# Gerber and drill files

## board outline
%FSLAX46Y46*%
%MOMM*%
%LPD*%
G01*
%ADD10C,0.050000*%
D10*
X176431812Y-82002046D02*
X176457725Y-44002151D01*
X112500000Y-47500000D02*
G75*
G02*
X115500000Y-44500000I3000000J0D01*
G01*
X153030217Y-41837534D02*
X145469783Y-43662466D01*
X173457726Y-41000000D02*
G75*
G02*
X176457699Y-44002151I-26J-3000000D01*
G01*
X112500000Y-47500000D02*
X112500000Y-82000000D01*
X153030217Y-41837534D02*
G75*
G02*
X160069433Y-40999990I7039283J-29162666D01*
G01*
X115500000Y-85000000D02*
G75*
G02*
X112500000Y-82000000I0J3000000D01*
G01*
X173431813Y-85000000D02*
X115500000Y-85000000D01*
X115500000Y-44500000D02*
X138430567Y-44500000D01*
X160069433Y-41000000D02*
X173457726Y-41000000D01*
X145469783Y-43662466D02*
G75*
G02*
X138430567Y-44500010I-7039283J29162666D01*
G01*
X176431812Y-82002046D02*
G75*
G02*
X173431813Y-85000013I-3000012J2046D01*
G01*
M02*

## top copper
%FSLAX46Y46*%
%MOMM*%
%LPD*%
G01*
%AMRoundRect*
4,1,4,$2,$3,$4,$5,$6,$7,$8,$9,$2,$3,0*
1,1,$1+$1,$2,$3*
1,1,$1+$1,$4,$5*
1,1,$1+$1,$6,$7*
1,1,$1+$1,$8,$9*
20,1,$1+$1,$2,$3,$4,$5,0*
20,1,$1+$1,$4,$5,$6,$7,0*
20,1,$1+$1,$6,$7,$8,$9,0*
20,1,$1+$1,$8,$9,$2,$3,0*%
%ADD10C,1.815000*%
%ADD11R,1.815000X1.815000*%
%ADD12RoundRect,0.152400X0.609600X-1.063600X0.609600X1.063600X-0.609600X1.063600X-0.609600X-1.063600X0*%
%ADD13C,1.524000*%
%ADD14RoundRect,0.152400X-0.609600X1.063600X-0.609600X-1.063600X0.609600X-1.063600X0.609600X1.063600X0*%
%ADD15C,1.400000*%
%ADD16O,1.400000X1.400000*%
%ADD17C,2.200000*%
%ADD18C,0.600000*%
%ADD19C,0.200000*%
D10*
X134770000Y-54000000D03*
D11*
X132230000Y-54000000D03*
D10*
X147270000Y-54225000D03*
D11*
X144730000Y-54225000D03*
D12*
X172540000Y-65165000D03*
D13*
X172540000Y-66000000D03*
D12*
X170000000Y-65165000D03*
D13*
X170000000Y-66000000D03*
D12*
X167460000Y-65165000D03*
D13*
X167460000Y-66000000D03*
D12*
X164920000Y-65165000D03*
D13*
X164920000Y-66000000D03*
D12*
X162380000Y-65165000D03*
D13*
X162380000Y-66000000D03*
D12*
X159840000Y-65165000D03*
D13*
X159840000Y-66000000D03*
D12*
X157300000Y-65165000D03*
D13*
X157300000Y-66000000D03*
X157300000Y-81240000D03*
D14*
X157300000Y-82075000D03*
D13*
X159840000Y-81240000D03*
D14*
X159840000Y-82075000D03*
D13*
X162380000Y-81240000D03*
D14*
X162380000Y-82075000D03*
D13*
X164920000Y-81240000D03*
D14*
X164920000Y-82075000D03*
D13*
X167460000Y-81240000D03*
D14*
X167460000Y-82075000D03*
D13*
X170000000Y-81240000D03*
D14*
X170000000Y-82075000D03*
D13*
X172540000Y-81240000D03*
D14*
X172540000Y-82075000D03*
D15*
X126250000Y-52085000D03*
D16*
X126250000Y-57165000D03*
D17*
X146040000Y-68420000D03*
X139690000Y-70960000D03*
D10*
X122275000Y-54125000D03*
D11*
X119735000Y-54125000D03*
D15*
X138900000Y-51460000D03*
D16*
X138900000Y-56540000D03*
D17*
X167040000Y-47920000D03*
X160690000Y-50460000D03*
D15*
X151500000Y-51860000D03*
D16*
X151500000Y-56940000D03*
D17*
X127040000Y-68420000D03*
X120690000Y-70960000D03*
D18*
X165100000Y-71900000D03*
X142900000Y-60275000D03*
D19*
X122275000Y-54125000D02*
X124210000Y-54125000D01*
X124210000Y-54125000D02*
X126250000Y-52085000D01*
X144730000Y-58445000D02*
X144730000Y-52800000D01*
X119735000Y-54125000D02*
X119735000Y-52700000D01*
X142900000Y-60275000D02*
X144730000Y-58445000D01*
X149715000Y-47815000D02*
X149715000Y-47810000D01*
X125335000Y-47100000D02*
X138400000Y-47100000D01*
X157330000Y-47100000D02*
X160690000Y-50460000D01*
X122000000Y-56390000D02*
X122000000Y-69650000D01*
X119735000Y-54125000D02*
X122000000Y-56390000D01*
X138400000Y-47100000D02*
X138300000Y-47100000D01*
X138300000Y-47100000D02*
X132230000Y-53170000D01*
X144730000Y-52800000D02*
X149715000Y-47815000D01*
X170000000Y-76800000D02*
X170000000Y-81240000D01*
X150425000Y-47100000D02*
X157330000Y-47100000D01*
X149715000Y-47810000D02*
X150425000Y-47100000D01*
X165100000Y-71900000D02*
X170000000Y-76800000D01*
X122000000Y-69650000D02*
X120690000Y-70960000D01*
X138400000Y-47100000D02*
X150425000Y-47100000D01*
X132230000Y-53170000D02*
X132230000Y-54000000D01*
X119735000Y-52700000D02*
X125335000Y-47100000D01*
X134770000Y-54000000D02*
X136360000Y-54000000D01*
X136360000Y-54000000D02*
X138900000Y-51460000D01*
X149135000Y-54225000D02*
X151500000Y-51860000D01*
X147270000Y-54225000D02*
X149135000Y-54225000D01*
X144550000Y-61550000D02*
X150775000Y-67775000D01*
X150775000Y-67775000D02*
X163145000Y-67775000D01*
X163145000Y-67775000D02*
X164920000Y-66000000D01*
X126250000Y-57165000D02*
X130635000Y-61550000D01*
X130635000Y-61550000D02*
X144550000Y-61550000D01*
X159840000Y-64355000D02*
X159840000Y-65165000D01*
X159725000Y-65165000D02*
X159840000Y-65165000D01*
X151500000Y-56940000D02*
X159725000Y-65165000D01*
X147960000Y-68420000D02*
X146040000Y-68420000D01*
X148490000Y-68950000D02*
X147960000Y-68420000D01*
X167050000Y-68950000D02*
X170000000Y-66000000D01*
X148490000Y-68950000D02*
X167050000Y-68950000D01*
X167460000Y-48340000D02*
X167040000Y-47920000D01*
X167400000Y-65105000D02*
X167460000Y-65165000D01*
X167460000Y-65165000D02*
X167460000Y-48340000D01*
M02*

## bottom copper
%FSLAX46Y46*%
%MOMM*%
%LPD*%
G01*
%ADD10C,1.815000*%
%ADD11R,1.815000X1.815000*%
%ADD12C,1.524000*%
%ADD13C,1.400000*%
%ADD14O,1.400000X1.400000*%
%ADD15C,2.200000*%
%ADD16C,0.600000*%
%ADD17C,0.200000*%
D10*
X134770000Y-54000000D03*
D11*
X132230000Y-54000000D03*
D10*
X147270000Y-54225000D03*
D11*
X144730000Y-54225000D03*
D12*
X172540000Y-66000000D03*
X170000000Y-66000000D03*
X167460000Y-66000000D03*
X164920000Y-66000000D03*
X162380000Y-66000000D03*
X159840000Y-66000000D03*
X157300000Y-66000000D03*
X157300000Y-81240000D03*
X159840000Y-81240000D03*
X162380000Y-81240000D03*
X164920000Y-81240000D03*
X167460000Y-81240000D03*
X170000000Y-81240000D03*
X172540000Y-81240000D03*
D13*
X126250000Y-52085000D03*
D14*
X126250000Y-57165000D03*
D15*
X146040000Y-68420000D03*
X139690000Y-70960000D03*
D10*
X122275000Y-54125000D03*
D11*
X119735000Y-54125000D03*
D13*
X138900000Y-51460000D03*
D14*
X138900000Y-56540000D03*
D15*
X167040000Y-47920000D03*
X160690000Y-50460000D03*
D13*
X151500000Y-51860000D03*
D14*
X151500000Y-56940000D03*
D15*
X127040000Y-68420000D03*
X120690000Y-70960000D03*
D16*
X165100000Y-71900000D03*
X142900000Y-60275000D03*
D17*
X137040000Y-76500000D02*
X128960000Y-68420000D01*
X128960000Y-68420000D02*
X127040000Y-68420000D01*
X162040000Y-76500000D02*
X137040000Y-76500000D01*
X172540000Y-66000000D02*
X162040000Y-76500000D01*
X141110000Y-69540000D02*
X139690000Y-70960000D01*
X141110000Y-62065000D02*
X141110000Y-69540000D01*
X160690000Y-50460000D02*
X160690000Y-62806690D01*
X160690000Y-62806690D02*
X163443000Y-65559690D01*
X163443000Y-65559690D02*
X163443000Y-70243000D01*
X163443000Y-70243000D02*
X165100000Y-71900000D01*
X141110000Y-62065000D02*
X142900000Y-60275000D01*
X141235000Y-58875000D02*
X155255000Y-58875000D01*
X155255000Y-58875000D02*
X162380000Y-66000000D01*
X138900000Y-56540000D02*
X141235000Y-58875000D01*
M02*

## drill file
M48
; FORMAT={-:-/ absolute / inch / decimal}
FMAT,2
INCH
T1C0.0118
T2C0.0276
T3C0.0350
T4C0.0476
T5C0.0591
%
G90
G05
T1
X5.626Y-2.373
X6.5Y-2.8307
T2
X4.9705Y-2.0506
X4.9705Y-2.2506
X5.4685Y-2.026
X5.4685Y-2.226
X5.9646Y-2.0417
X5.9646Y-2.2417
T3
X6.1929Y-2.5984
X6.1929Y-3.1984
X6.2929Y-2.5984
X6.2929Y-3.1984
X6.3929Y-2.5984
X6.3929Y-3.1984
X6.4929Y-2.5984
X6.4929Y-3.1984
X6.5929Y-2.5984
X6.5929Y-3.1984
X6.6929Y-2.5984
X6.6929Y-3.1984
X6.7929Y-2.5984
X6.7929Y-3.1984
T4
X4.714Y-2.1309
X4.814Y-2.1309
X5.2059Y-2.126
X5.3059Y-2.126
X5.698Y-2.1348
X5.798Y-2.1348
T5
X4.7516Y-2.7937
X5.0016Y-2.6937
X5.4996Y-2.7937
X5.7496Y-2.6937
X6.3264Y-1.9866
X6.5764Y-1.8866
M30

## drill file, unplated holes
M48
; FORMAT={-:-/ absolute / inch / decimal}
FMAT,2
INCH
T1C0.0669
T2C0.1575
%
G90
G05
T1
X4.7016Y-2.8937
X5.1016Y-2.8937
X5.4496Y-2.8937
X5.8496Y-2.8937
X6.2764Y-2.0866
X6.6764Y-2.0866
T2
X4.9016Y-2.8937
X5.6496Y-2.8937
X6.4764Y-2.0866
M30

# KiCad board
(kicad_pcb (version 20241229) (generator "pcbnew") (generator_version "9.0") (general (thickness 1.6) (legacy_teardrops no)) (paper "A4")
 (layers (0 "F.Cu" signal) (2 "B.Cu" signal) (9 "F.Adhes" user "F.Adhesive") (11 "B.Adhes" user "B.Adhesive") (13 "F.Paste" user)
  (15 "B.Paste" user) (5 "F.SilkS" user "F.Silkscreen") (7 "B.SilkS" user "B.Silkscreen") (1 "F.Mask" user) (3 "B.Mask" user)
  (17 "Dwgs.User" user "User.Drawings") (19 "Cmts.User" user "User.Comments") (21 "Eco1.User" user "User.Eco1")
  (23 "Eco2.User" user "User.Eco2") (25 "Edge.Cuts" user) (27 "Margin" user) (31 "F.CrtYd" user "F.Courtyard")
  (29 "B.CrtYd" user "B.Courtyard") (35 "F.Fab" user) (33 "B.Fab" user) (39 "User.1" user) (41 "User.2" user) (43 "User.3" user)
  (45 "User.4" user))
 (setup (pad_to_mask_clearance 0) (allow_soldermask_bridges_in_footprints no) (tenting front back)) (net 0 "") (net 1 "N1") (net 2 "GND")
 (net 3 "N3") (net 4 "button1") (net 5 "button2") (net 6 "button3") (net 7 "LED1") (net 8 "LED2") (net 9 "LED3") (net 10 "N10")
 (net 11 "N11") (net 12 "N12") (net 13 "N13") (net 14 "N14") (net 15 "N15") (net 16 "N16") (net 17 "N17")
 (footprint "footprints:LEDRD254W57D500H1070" (layer "F.Cu") (at 133.5 54)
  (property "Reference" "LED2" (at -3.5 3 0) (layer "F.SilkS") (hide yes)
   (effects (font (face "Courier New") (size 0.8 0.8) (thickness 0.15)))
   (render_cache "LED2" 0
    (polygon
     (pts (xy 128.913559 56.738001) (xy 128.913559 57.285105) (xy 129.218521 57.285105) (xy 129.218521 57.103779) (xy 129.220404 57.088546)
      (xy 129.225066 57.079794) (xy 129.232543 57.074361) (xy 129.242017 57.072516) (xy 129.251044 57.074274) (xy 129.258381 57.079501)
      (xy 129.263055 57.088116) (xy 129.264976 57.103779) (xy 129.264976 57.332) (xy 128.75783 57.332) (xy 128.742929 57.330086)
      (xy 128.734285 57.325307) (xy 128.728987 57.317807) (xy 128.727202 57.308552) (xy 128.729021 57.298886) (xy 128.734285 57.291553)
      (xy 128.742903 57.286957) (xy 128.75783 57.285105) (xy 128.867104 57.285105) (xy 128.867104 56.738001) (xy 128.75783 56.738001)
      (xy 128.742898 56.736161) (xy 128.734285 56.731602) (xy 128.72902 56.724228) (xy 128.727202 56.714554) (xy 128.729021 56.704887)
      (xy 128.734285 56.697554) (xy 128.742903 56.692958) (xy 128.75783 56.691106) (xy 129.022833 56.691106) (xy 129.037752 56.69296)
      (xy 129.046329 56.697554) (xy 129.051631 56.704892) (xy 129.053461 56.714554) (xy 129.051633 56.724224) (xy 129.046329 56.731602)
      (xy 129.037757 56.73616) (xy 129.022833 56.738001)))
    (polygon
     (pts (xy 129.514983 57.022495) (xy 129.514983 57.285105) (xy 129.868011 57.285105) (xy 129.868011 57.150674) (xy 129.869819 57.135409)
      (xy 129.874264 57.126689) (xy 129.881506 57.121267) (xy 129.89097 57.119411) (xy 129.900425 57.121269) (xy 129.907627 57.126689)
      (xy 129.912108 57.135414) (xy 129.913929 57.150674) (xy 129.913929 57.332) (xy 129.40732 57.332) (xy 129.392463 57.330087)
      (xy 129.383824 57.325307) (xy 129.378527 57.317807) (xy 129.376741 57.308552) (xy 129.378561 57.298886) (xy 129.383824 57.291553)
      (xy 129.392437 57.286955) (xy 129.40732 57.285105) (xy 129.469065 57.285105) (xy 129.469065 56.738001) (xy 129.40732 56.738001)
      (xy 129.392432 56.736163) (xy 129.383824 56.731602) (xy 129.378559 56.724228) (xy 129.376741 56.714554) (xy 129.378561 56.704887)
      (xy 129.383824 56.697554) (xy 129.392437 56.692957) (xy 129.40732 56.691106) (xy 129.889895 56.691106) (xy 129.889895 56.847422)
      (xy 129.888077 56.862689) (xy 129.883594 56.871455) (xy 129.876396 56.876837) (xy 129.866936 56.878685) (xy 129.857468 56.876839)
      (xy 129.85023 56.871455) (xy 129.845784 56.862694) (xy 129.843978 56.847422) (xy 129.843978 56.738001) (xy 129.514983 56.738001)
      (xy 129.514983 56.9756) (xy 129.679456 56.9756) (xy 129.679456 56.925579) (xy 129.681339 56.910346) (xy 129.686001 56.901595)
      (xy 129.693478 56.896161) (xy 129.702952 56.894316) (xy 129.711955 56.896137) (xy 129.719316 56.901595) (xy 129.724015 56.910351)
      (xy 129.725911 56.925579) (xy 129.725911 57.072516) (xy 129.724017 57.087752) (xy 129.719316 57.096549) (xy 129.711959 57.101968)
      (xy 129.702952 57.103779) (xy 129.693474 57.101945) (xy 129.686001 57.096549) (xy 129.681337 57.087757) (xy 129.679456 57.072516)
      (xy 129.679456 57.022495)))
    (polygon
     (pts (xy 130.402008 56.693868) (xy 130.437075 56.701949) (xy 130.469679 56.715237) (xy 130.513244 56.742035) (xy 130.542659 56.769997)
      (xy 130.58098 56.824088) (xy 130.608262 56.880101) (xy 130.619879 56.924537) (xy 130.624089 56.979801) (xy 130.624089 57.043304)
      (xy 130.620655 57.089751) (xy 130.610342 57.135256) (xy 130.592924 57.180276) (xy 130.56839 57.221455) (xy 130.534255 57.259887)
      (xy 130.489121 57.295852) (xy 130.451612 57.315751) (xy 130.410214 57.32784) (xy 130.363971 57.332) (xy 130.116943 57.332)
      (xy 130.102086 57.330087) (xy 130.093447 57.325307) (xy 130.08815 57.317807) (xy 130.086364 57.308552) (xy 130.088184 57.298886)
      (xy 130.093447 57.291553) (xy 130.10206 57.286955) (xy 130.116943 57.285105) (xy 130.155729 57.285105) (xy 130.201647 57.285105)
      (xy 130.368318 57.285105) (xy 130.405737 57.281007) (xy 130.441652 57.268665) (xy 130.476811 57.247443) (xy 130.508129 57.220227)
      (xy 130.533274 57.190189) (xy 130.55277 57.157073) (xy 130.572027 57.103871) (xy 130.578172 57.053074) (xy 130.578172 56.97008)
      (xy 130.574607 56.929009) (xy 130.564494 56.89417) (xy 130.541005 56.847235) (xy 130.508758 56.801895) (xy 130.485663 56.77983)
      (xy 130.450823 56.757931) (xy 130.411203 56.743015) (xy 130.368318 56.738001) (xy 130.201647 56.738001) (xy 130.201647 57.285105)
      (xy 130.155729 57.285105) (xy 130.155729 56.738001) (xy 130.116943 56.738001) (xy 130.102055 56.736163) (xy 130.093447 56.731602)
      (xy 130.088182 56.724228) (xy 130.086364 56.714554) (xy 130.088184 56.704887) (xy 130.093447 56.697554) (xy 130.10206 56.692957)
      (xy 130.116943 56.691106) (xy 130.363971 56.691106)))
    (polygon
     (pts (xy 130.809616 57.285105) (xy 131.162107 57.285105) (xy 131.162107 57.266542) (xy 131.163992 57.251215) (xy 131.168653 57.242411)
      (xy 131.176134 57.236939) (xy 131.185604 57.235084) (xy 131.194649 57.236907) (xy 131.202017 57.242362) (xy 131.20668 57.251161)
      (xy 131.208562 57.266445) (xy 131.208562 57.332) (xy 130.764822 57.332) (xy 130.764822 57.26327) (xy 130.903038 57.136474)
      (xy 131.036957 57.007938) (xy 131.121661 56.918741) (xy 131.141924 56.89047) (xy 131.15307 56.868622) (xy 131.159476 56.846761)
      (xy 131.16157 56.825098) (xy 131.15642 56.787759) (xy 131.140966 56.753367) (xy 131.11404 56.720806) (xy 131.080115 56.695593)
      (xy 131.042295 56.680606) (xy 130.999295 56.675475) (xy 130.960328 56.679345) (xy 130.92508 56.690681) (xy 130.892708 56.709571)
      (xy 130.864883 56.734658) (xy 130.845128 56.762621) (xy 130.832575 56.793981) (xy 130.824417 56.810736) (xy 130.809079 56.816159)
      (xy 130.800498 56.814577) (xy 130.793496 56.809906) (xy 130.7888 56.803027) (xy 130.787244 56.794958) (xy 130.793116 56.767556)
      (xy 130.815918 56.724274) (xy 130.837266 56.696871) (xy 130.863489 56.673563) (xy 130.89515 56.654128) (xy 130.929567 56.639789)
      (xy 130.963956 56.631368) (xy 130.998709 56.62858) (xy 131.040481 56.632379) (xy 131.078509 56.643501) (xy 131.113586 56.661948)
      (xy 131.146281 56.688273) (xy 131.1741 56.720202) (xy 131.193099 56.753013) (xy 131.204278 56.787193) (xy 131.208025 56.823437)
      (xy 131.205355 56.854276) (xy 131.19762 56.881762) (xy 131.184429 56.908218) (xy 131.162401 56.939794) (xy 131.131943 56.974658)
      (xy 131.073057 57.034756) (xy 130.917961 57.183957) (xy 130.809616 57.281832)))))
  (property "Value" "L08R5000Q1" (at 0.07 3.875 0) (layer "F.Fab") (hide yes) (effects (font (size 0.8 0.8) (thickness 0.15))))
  (pad "A" thru_hole circle (at 1.27 0) (size 1.815 1.815) (drill 1.21) (layers "*.Cu" "*.Mask") (remove_unused_layers no) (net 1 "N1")
   (solder_mask_margin 0.102))
  (pad "C" thru_hole rect (at -1.27 0) (size 1.815 1.815) (drill 1.21) (layers "*.Cu" "*.Mask") (remove_unused_layers no) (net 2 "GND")
   (solder_mask_margin 0.102)))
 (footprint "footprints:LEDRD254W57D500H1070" (layer "F.Cu") (at 146 54.225)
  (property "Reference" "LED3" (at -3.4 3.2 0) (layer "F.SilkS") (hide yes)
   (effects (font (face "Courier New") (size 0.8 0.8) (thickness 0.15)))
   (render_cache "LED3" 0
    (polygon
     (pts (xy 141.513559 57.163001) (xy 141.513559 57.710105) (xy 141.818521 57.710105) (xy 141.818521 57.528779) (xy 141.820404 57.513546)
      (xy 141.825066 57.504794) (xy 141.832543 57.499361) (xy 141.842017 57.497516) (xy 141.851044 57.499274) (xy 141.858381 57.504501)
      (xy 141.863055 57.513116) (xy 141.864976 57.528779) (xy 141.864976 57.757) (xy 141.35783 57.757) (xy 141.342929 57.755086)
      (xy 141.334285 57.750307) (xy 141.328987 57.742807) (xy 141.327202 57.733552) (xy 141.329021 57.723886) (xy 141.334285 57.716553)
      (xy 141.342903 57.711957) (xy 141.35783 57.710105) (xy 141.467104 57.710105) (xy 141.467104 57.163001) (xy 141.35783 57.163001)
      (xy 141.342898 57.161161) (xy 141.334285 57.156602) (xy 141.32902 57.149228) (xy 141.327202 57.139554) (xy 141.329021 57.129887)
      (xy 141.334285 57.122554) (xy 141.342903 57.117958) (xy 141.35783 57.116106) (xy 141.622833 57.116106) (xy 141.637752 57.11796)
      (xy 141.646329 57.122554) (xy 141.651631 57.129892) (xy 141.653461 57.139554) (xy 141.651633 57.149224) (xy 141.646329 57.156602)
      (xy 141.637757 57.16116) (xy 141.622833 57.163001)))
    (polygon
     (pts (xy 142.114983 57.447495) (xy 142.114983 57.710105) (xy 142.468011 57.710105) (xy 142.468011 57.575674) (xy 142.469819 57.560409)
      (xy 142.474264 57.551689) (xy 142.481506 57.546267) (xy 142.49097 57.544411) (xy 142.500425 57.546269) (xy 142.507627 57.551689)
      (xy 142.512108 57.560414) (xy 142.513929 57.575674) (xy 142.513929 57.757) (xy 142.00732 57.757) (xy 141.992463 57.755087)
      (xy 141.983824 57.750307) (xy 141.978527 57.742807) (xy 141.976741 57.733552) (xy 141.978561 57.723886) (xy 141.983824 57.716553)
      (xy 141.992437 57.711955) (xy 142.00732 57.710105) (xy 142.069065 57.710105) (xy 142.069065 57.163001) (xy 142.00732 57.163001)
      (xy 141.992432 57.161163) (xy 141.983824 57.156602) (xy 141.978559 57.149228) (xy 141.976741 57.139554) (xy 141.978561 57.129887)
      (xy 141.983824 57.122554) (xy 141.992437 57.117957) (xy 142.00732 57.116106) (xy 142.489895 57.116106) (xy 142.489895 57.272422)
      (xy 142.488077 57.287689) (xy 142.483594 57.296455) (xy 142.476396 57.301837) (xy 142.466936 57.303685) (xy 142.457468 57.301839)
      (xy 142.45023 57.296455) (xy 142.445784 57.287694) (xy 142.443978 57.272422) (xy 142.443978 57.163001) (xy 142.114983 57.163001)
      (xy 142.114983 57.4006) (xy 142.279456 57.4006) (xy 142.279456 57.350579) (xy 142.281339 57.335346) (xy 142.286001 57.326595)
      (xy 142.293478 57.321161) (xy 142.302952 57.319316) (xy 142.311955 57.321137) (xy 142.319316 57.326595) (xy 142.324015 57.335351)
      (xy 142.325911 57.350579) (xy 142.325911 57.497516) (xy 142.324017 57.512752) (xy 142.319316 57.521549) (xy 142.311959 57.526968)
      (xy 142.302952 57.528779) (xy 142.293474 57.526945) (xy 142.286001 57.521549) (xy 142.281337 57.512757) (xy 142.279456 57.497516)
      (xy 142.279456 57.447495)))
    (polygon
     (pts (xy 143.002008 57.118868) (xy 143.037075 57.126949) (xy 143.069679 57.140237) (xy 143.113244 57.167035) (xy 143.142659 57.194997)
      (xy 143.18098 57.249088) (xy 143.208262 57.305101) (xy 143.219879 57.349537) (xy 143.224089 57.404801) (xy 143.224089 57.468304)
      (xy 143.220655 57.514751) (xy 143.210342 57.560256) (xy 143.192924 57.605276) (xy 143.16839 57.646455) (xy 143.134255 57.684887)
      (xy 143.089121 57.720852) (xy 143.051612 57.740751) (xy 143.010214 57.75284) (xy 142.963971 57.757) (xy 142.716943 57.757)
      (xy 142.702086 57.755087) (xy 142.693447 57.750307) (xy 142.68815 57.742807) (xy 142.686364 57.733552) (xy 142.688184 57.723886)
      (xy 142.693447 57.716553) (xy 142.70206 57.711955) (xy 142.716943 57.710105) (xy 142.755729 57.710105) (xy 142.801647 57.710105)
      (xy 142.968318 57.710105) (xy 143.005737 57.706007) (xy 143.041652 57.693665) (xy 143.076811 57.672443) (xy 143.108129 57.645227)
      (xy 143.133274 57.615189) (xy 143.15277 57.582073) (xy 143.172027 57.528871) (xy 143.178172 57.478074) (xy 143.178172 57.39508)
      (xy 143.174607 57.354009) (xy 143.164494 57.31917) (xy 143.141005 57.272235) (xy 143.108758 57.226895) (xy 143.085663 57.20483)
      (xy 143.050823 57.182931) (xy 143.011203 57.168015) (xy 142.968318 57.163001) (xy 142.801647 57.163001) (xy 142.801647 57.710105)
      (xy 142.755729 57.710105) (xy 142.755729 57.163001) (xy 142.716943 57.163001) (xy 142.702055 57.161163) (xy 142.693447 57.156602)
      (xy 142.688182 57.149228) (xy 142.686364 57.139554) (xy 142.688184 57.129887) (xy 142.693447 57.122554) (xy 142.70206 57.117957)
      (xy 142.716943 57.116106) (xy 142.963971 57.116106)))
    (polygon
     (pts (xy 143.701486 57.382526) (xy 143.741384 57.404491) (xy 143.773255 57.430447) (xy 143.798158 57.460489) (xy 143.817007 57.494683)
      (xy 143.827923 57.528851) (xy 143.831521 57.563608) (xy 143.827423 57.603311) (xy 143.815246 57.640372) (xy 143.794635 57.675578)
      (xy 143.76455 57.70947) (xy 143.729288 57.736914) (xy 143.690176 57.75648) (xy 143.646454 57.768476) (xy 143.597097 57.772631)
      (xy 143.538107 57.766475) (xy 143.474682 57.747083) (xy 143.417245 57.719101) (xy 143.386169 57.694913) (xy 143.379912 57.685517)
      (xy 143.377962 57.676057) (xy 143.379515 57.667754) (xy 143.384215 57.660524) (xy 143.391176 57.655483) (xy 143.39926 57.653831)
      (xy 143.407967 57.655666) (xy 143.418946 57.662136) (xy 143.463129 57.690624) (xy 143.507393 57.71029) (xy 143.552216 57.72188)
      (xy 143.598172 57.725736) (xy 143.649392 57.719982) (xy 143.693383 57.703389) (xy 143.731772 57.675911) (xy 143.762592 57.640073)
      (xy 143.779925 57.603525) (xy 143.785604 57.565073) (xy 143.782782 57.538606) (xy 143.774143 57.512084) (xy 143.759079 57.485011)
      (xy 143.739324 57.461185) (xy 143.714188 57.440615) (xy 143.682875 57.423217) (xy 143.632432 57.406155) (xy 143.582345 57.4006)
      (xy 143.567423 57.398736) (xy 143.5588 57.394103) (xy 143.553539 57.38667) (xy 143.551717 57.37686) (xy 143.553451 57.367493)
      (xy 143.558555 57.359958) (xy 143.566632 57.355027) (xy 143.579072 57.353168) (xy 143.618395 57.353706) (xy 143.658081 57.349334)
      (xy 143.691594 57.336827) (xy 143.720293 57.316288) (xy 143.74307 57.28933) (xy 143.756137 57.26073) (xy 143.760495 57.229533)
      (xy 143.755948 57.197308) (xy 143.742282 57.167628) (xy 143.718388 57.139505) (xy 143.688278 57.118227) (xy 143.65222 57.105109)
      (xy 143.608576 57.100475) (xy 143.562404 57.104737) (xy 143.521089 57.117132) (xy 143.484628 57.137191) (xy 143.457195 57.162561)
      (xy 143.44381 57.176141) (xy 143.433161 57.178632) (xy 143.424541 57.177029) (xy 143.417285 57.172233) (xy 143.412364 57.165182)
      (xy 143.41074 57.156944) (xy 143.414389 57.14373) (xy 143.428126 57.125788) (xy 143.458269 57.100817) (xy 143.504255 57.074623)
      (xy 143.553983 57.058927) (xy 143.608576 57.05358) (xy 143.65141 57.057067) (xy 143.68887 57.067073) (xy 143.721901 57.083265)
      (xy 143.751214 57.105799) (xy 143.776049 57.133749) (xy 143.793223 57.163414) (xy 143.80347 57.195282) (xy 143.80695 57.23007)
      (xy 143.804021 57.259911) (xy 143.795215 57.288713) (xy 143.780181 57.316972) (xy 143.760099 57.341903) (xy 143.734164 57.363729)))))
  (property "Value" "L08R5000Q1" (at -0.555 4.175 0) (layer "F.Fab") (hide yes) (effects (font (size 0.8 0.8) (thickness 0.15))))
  (pad "A" thru_hole circle (at 1.27 0) (size 1.815 1.815) (drill 1.21) (layers "*.Cu" "*.Mask") (remove_unused_layers no) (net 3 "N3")
   (solder_mask_margin 0.102))
  (pad "C" thru_hole rect (at -1.27 0) (size 1.815 1.815) (drill 1.21) (layers "*.Cu" "*.Mask") (remove_unused_layers no) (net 2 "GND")
   (solder_mask_margin 0.102)))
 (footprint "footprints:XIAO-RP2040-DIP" (layer "F.Cu") (at 164.92 73.62 -90)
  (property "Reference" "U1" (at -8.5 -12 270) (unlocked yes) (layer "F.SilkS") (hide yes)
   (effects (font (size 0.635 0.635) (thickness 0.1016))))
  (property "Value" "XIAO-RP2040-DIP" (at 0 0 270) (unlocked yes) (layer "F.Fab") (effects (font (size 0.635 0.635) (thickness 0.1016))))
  (pad "1" smd roundrect (at -8.455 -7.62 90) (size 2.432 1.524) (layers "F.Cu" "F.Mask") (roundrect_rratio 0.1) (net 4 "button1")
   (thermal_bridge_angle 45))
  (pad "1" thru_hole circle (at -7.62 -7.62 90) (size 1.524 1.524) (drill 0.889) (layers "*.Cu" "*.Mask") (remove_unused_layers no)
   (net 4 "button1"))
  (pad "2" smd roundrect (at -8.455 -5.08 90) (size 2.432 1.524) (layers "F.Cu" "F.Mask") (roundrect_rratio 0.1) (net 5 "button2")
   (thermal_bridge_angle 45))
  (pad "2" thru_hole circle (at -7.62 -5.08 90) (size 1.524 1.524) (drill 0.889) (layers "*.Cu" "*.Mask") (remove_unused_layers no)
   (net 5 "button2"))
  (pad "3" smd roundrect (at -8.455 -2.54 90) (size 2.432 1.524) (layers "F.Cu" "F.Mask") (roundrect_rratio 0.1) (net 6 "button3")
   (thermal_bridge_angle 45))
  (pad "3" thru_hole circle (at -7.62 -2.54 90) (size 1.524 1.524) (drill 0.889) (layers "*.Cu" "*.Mask") (remove_unused_layers no)
   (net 6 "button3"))
  (pad "4" smd roundrect (at -8.455 0 90) (size 2.432 1.524) (layers "F.Cu" "F.Mask") (roundrect_rratio 0.1) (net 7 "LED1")
   (thermal_bridge_angle 45))
  (pad "4" thru_hole circle (at -7.62 0 90) (size 1.524 1.524) (drill 0.889) (layers "*.Cu" "*.Mask") (remove_unused_layers no)
   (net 7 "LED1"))
  (pad "5" smd roundrect (at -8.455 2.54 90) (size 2.432 1.524) (layers "F.Cu" "F.Mask") (roundrect_rratio 0.1) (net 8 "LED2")
   (thermal_bridge_angle 45))
  (pad "5" thru_hole circle (at -7.62 2.54 90) (size 1.524 1.524) (drill 0.889) (layers "*.Cu" "*.Mask") (remove_unused_layers no)
   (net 8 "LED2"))
  (pad "6" smd roundrect (at -8.455 5.08 90) (size 2.432 1.524) (layers "F.Cu" "F.Mask") (roundrect_rratio 0.1) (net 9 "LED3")
   (thermal_bridge_angle 45))
  (pad "6" thru_hole circle (at -7.62 5.08 90) (size 1.524 1.524) (drill 0.889) (layers "*.Cu" "*.Mask") (remove_unused_layers no)
   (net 9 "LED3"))
  (pad "7" smd roundrect (at -8.455 7.62 90) (size 2.432 1.524) (layers "F.Cu" "F.Mask") (roundrect_rratio 0.1) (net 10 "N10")
   (thermal_bridge_angle 45))
  (pad "7" thru_hole circle (at -7.62 7.62 90) (size 1.524 1.524) (drill 0.889) (layers "*.Cu" "*.Mask") (remove_unused_layers no)
   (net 10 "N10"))
  (pad "8" thru_hole circle (at 7.62 7.62 270) (size 1.524 1.524) (drill 0.889) (layers "*.Cu" "*.Mask") (remove_unused_layers no)
   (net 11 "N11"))
  (pad "8" smd roundrect (at 8.455 7.62 270) (size 2.432 1.524) (layers "F.Cu" "F.Mask") (roundrect_rratio 0.1) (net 11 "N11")
   (thermal_bridge_angle 45))
  (pad "9" thru_hole circle (at 7.62 5.08 270) (size 1.524 1.524) (drill 0.889) (layers "*.Cu" "*.Mask") (remove_unused_layers no)
   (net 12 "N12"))
  (pad "9" smd roundrect (at 8.455 5.08 270) (size 2.432 1.524) (layers "F.Cu" "F.Mask") (roundrect_rratio 0.1) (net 12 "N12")
   (thermal_bridge_angle 45))
  (pad "10" thru_hole circle (at 7.62 2.54 270) (size 1.524 1.524) (drill 0.889) (layers "*.Cu" "*.Mask") (remove_unused_layers no)
   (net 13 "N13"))
  (pad "10" smd roundrect (at 8.455 2.54 270) (size 2.432 1.524) (layers "F.Cu" "F.Mask") (roundrect_rratio 0.1) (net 13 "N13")
   (thermal_bridge_angle 45))
  (pad "11" thru_hole circle (at 7.62 0 270) (size 1.524 1.524) (drill 0.889) (layers "*.Cu" "*.Mask") (remove_unused_layers no)
   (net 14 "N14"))
  (pad "11" smd roundrect (at 8.455 0 270) (size 2.432 1.524) (layers "F.Cu" "F.Mask") (roundrect_rratio 0.1) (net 14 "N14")
   (thermal_bridge_angle 45))
  (pad "12" thru_hole circle (at 7.62 -2.54 270) (size 1.524 1.524) (drill 0.889) (layers "*.Cu" "*.Mask") (remove_unused_layers no)
   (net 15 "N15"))
  (pad "12" smd roundrect (at 8.455 -2.54 270) (size 2.432 1.524) (layers "F.Cu" "F.Mask") (roundrect_rratio 0.1) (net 15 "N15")
   (thermal_bridge_angle 45))
  (pad "13" thru_hole circle (at 7.62 -5.08 270) (size 1.524 1.524) (drill 0.889) (layers "*.Cu" "*.Mask") (remove_unused_layers no)
   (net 2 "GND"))
  (pad "13" smd roundrect (at 8.455 -5.08 270) (size 2.432 1.524) (layers "F.Cu" "F.Mask") (roundrect_rratio 0.1) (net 2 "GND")
   (thermal_bridge_angle 45))
  (pad "14" thru_hole circle (at 7.62 -7.62 270) (size 1.524 1.524) (drill 0.889) (layers "*.Cu" "*.Mask") (remove_unused_layers no)
   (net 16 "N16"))
  (pad "14" smd roundrect (at 8.455 -7.62 270) (size 2.432 1.524) (layers "F.Cu" "F.Mask") (roundrect_rratio 0.1) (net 16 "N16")
   (thermal_bridge_angle 45)))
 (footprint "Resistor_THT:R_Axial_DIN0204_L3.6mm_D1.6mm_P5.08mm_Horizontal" (layer "F.Cu") (at 126.25 52.085 -90)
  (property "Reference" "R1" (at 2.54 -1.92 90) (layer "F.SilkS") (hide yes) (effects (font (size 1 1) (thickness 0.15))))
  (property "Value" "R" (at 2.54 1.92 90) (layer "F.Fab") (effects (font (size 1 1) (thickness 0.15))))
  (pad "1" thru_hole circle (at 0 0 270) (size 1.4 1.4) (drill 0.7) (layers "*.Cu" "*.Mask") (remove_unused_layers no) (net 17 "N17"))
  (pad "2" thru_hole oval (at 5.08 0 270) (size 1.4 1.4) (drill 0.7) (layers "*.Cu" "*.Mask") (remove_unused_layers no) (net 7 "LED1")))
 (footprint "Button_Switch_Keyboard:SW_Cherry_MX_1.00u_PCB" (layer "F.Cu") (at 146.04 68.42)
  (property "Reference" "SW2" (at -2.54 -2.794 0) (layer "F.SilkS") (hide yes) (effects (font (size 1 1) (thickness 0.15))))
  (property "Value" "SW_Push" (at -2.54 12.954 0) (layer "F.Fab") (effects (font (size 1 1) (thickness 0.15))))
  (pad "" np_thru_hole circle (at -7.62 5.08) (size 1.7 1.7) (drill 1.7) (layers "*.Cu" "*.Mask"))
  (pad "" np_thru_hole circle (at -2.54 5.08) (size 4 4) (drill 4) (layers "*.Cu" "*.Mask"))
  (pad "" np_thru_hole circle (at 2.54 5.08) (size 1.7 1.7) (drill 1.7) (layers "*.Cu" "*.Mask"))
  (pad "1" thru_hole circle (at 0 0) (size 2.2 2.2) (drill 1.5) (layers "*.Cu" "*.Mask") (remove_unused_layers no) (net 5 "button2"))
  (pad "2" thru_hole circle (at -6.35 2.54) (size 2.2 2.2) (drill 1.5) (layers "*.Cu" "*.Mask") (remove_unused_layers no) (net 2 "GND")))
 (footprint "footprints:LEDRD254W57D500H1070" (layer "F.Cu") (at 121.005 54.125)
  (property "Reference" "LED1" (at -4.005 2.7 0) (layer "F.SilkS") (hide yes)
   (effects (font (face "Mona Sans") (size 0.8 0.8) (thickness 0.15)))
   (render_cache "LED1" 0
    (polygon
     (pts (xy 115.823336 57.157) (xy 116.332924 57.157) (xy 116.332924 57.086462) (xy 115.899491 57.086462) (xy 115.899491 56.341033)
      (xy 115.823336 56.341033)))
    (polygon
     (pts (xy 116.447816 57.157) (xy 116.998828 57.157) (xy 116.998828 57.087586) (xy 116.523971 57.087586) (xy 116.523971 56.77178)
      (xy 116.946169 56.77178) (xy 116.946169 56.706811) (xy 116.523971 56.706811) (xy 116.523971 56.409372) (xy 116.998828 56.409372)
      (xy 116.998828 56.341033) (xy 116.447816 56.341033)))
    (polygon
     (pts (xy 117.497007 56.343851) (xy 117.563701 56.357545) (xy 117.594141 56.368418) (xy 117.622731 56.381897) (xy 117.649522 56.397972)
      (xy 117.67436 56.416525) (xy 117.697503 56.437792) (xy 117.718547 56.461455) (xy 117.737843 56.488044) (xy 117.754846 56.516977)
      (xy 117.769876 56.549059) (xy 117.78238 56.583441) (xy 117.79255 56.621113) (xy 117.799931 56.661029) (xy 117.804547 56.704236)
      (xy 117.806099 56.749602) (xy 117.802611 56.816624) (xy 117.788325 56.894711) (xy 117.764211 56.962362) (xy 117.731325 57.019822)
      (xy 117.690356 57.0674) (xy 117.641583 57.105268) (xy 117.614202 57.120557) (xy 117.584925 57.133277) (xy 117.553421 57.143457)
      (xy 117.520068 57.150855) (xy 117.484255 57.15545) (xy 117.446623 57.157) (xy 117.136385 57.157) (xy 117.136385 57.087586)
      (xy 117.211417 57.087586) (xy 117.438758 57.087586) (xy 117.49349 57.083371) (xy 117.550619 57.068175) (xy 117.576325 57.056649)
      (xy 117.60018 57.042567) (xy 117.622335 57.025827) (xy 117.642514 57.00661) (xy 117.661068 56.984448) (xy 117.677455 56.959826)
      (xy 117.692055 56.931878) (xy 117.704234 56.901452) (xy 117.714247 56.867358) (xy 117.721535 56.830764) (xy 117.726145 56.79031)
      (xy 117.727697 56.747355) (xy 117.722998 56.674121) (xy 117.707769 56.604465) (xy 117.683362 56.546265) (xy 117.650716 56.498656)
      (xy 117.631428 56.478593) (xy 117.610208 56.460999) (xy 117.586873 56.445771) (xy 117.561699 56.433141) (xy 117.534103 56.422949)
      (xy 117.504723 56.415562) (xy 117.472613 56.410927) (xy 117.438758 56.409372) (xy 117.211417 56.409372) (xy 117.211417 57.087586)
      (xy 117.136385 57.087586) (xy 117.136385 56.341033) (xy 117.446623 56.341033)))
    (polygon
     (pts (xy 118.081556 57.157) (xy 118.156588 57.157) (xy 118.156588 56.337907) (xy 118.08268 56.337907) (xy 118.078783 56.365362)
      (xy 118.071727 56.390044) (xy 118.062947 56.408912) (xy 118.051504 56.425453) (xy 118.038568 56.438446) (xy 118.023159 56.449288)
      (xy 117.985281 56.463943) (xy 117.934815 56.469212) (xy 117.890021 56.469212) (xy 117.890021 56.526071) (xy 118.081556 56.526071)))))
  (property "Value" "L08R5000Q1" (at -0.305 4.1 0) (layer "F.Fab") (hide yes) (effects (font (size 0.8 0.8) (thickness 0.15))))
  (pad "A" thru_hole circle (at 1.27 0) (size 1.815 1.815) (drill 1.21) (layers "*.Cu" "*.Mask") (remove_unused_layers no) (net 17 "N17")
   (solder_mask_margin 0.102))
  (pad "C" thru_hole rect (at -1.27 0) (size 1.815 1.815) (drill 1.21) (layers "*.Cu" "*.Mask") (remove_unused_layers no) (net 2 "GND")
   (solder_mask_margin 0.102)))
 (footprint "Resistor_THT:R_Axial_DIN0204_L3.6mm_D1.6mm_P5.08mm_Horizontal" (layer "F.Cu") (at 138.9 51.46 -90)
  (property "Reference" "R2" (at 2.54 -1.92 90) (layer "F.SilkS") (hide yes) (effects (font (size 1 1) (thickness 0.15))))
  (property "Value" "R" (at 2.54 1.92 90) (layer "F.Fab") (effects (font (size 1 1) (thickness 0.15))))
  (pad "1" thru_hole circle (at 0 0 270) (size 1.4 1.4) (drill 0.7) (layers "*.Cu" "*.Mask") (remove_unused_layers no) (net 1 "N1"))
  (pad "2" thru_hole oval (at 5.08 0 270) (size 1.4 1.4) (drill 0.7) (layers "*.Cu" "*.Mask") (remove_unused_layers no) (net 8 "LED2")))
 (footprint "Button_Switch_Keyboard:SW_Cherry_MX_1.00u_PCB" (layer "F.Cu") (at 167.04 47.92)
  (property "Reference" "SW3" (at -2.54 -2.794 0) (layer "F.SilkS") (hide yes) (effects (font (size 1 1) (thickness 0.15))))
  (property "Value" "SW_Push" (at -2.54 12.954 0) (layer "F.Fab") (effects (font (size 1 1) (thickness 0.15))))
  (pad "" np_thru_hole circle (at -7.62 5.08) (size 1.7 1.7) (drill 1.7) (layers "*.Cu" "*.Mask"))
  (pad "" np_thru_hole circle (at -2.54 5.08) (size 4 4) (drill 4) (layers "*.Cu" "*.Mask"))
  (pad "" np_thru_hole circle (at 2.54 5.08) (size 1.7 1.7) (drill 1.7) (layers "*.Cu" "*.Mask"))
  (pad "1" thru_hole circle (at 0 0) (size 2.2 2.2) (drill 1.5) (layers "*.Cu" "*.Mask") (remove_unused_layers no) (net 6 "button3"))
  (pad "2" thru_hole circle (at -6.35 2.54) (size 2.2 2.2) (drill 1.5) (layers "*.Cu" "*.Mask") (remove_unused_layers no) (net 2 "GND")))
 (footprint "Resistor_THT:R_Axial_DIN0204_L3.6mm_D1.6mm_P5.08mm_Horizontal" (layer "F.Cu") (at 151.5 51.86 -90)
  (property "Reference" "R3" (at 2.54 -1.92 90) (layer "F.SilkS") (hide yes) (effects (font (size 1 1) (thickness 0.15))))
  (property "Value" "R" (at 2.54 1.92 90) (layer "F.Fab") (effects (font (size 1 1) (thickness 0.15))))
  (pad "1" thru_hole circle (at 0 0 270) (size 1.4 1.4) (drill 0.7) (layers "*.Cu" "*.Mask") (remove_unused_layers no) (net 3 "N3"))
  (pad "2" thru_hole oval (at 5.08 0 270) (size 1.4 1.4) (drill 0.7) (layers "*.Cu" "*.Mask") (remove_unused_layers no) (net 9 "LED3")))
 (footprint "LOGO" (layer "F.Cu") (at 116 50.2)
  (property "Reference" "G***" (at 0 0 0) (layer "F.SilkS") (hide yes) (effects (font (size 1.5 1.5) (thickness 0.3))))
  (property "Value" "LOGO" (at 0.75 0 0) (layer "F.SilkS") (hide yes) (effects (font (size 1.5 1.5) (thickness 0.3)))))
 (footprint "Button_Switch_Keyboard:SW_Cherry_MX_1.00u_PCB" (layer "F.Cu") (at 127.04 68.42)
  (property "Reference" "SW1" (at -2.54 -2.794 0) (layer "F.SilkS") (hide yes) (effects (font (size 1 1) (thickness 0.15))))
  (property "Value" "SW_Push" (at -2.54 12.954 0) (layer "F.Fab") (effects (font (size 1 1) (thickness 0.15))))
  (pad "" np_thru_hole circle (at -7.62 5.08) (size 1.7 1.7) (drill 1.7) (layers "*.Cu" "*.Mask"))
  (pad "" np_thru_hole circle (at -2.54 5.08) (size 4 4) (drill 4) (layers "*.Cu" "*.Mask"))
  (pad "" np_thru_hole circle (at 2.54 5.08) (size 1.7 1.7) (drill 1.7) (layers "*.Cu" "*.Mask"))
  (pad "1" thru_hole circle (at 0 0) (size 2.2 2.2) (drill 1.5) (layers "*.Cu" "*.Mask") (remove_unused_layers no) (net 4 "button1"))
  (pad "2" thru_hole circle (at -6.35 2.54) (size 2.2 2.2) (drill 1.5) (layers "*.Cu" "*.Mask") (remove_unused_layers no) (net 2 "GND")))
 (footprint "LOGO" (layer "F.Cu") (at 121 49.5)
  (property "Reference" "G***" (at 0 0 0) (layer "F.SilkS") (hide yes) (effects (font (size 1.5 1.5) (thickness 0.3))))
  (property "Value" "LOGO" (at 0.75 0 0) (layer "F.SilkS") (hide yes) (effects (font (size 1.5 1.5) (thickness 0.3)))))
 (gr_line (start 176.431812 82.002046) (end 176.457725 44.002151) (stroke (width 0.05) (type default)) (layer "Edge.Cuts"))
 (gr_arc (start 112.5 47.5) (mid 113.37868 45.37868) (end 115.5 44.5) (stroke (width 0.05) (type default)) (layer "Edge.Cuts"))
 (gr_line (start 153.030217 41.837534) (end 145.469783 43.662466) (stroke (width 0.05) (type default)) (layer "Edge.Cuts"))
 (gr_arc (start 173.457726 41) (mid 175.57979 41.879449) (end 176.457725 44.002151) (stroke (width 0.05) (type default)) (layer "Edge.Cuts"))
 (gr_line (start 112.5 47.5) (end 112.5 82) (stroke (width 0.05) (type default)) (layer "Edge.Cuts"))
 (gr_arc (start 153.030217 41.837534) (mid 156.525 41.210121) (end 160.069433 41) (stroke (width 0.05) (type default)) (layer "Edge.Cuts"))
 (gr_arc (start 115.5 85) (mid 113.37868 84.12132) (end 112.5 82) (stroke (width 0.05) (type default)) (layer "Edge.Cuts"))
 (gr_line (start 173.431813 85) (end 115.5 85) (stroke (width 0.05) (type default)) (layer "Edge.Cuts"))
 (gr_line (start 115.5 44.5) (end 138.430567 44.5) (stroke (width 0.05) (type default)) (layer "Edge.Cuts"))
 (gr_line (start 160.069433 41) (end 173.457726 41) (stroke (width 0.05) (type default)) (layer "Edge.Cuts"))
 (gr_arc (start 145.469783 43.662466) (mid 141.975 44.289879) (end 138.430567 44.5) (stroke (width 0.05) (type default)) (layer "Edge.Cuts"))
 (gr_arc (start 176.431812 82.002046) (mid 175.55241 84.122043) (end 173.431813 85) (stroke (width 0.05) (type default)) (layer "Edge.Cuts"))
 (segment (start 122.275 54.125) (end 124.21 54.125) (width 0.2) (layer "F.Cu") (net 17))
 (segment (start 124.21 54.125) (end 126.25 52.085) (width 0.2) (layer "F.Cu") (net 17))
 (segment (start 144.73 58.445) (end 144.73 52.8) (width 0.2) (layer "F.Cu") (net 2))
 (segment (start 119.735 54.125) (end 119.735 52.7) (width 0.2) (layer "F.Cu") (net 2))
 (segment (start 142.9 60.275) (end 144.73 58.445) (width 0.2) (layer "F.Cu") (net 2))
 (segment (start 149.715 47.815) (end 149.715 47.81) (width 0.2) (layer "F.Cu") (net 2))
 (segment (start 125.335 47.1) (end 138.4 47.1) (width 0.2) (layer "F.Cu") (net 2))
 (segment (start 157.33 47.1) (end 160.69 50.46) (width 0.2) (layer "F.Cu") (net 2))
 (segment (start 122 56.39) (end 122 69.65) (width 0.2) (layer "F.Cu") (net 2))
 (segment (start 119.735 54.125) (end 122 56.39) (width 0.2) (layer "F.Cu") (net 2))
 (segment (start 138.4 47.1) (end 138.3 47.1) (width 0.2) (layer "F.Cu") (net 2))
 (segment (start 138.3 47.1) (end 132.23 53.17) (width 0.2) (layer "F.Cu") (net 2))
 (segment (start 144.73 52.8) (end 149.715 47.815) (width 0.2) (layer "F.Cu") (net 2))
 (segment (start 170 76.8) (end 170 81.24) (width 0.2) (layer "F.Cu") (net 2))
 (segment (start 150.425 47.1) (end 157.33 47.1) (width 0.2) (layer "F.Cu") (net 2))
 (segment (start 149.715 47.81) (end 150.425 47.1) (width 0.2) (layer "F.Cu") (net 2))
 (segment (start 165.1 71.9) (end 170 76.8) (width 0.2) (layer "F.Cu") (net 2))
 (segment (start 122 69.65) (end 120.69 70.96) (width 0.2) (layer "F.Cu") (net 2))
 (segment (start 138.4 47.1) (end 150.425 47.1) (width 0.2) (layer "F.Cu") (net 2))
 (segment (start 132.23 53.17) (end 132.23 54) (width 0.2) (layer "F.Cu") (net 2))
 (segment (start 119.735 52.7) (end 125.335 47.1) (width 0.2) (layer "F.Cu") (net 2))
 (via (at 165.1 71.9) (size 0.6) (drill 0.3) (layers "F.Cu" "B.Cu") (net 2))
 (via (at 142.9 60.275) (size 0.6) (drill 0.3) (layers "F.Cu" "B.Cu") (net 2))
 (segment (start 141.11 69.54) (end 139.69 70.96) (width 0.2) (layer "B.Cu") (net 2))
 (segment (start 141.11 62.065) (end 141.11 69.54) (width 0.2) (layer "B.Cu") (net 2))
 (segment (start 160.69 50.46) (end 160.69 62.80669) (width 0.2) (layer "B.Cu") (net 2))
 (segment (start 160.69 62.80669) (end 163.443 65.55969) (width 0.2) (layer "B.Cu") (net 2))
 (segment (start 163.443 65.55969) (end 163.443 70.243) (width 0.2) (layer "B.Cu") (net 2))
 (segment (start 163.443 70.243) (end 165.1 71.9) (width 0.2) (layer "B.Cu") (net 2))
 (segment (start 141.11 62.065) (end 142.9 60.275) (width 0.2) (layer "B.Cu") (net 2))
 (segment (start 134.77 54) (end 136.36 54) (width 0.2) (layer "F.Cu") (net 1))
 (segment (start 136.36 54) (end 138.9 51.46) (width 0.2) (layer "F.Cu") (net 1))
 (segment (start 149.135 54.225) (end 151.5 51.86) (width 0.2) (layer "F.Cu") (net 3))
 (segment (start 147.27 54.225) (end 149.135 54.225) (width 0.2) (layer "F.Cu") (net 3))
 (segment (start 144.55 61.55) (end 150.775 67.775) (width 0.2) (layer "F.Cu") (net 7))
 (segment (start 150.775 67.775) (end 163.145 67.775) (width 0.2) (layer "F.Cu") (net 7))
 (segment (start 163.145 67.775) (end 164.92 66) (width 0.2) (layer "F.Cu") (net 7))
 (segment (start 126.25 57.165) (end 130.635 61.55) (width 0.2) (layer "F.Cu") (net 7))
 (segment (start 130.635 61.55) (end 144.55 61.55) (width 0.2) (layer "F.Cu") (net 7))
 (segment (start 141.235 58.875) (end 155.255 58.875) (width 0.2) (layer "B.Cu") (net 8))
 (segment (start 155.255 58.875) (end 162.38 66) (width 0.2) (layer "B.Cu") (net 8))
 (segment (start 138.9 56.54) (end 141.235 58.875) (width 0.2) (layer "B.Cu") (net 8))
 (segment (start 159.84 64.355) (end 159.84 65.165) (width 0.2) (layer "F.Cu") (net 9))
 (segment (start 159.725 65.165) (end 159.84 65.165) (width 0.2) (layer "F.Cu") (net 9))
 (segment (start 151.5 56.94) (end 159.725 65.165) (width 0.2) (layer "F.Cu") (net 9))
 (segment (start 137.04 76.5) (end 128.96 68.42) (width 0.2) (layer "B.Cu") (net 4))
 (segment (start 172.54 66) (end 162.04 76.5) (width 0.2) (layer "B.Cu") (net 4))
 (segment (start 128.96 68.42) (end 127.04 68.42) (width 0.2) (layer "B.Cu") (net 4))
 (segment (start 162.04 76.5) (end 137.04 76.5) (width 0.2) (layer "B.Cu") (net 4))
 (segment (start 147.96 68.42) (end 146.04 68.42) (width 0.2) (layer "F.Cu") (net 5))
 (segment (start 148.49 68.95) (end 147.96 68.42) (width 0.2) (layer "F.Cu") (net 5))
 (segment (start 167.05 68.95) (end 170 66) (width 0.2) (layer "F.Cu") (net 5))
 (segment (start 148.49 68.95) (end 167.05 68.95) (width 0.2) (layer "F.Cu") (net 5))
 (segment (start 167.46 48.34) (end 167.04 47.92) (width 0.2) (layer "F.Cu") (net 6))
 (segment (start 167.4 65.105) (end 167.46 65.165) (width 0.2) (layer "F.Cu") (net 6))
 (segment (start 167.46 65.165) (end 167.46 48.34) (width 0.2) (layer "F.Cu") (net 6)))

